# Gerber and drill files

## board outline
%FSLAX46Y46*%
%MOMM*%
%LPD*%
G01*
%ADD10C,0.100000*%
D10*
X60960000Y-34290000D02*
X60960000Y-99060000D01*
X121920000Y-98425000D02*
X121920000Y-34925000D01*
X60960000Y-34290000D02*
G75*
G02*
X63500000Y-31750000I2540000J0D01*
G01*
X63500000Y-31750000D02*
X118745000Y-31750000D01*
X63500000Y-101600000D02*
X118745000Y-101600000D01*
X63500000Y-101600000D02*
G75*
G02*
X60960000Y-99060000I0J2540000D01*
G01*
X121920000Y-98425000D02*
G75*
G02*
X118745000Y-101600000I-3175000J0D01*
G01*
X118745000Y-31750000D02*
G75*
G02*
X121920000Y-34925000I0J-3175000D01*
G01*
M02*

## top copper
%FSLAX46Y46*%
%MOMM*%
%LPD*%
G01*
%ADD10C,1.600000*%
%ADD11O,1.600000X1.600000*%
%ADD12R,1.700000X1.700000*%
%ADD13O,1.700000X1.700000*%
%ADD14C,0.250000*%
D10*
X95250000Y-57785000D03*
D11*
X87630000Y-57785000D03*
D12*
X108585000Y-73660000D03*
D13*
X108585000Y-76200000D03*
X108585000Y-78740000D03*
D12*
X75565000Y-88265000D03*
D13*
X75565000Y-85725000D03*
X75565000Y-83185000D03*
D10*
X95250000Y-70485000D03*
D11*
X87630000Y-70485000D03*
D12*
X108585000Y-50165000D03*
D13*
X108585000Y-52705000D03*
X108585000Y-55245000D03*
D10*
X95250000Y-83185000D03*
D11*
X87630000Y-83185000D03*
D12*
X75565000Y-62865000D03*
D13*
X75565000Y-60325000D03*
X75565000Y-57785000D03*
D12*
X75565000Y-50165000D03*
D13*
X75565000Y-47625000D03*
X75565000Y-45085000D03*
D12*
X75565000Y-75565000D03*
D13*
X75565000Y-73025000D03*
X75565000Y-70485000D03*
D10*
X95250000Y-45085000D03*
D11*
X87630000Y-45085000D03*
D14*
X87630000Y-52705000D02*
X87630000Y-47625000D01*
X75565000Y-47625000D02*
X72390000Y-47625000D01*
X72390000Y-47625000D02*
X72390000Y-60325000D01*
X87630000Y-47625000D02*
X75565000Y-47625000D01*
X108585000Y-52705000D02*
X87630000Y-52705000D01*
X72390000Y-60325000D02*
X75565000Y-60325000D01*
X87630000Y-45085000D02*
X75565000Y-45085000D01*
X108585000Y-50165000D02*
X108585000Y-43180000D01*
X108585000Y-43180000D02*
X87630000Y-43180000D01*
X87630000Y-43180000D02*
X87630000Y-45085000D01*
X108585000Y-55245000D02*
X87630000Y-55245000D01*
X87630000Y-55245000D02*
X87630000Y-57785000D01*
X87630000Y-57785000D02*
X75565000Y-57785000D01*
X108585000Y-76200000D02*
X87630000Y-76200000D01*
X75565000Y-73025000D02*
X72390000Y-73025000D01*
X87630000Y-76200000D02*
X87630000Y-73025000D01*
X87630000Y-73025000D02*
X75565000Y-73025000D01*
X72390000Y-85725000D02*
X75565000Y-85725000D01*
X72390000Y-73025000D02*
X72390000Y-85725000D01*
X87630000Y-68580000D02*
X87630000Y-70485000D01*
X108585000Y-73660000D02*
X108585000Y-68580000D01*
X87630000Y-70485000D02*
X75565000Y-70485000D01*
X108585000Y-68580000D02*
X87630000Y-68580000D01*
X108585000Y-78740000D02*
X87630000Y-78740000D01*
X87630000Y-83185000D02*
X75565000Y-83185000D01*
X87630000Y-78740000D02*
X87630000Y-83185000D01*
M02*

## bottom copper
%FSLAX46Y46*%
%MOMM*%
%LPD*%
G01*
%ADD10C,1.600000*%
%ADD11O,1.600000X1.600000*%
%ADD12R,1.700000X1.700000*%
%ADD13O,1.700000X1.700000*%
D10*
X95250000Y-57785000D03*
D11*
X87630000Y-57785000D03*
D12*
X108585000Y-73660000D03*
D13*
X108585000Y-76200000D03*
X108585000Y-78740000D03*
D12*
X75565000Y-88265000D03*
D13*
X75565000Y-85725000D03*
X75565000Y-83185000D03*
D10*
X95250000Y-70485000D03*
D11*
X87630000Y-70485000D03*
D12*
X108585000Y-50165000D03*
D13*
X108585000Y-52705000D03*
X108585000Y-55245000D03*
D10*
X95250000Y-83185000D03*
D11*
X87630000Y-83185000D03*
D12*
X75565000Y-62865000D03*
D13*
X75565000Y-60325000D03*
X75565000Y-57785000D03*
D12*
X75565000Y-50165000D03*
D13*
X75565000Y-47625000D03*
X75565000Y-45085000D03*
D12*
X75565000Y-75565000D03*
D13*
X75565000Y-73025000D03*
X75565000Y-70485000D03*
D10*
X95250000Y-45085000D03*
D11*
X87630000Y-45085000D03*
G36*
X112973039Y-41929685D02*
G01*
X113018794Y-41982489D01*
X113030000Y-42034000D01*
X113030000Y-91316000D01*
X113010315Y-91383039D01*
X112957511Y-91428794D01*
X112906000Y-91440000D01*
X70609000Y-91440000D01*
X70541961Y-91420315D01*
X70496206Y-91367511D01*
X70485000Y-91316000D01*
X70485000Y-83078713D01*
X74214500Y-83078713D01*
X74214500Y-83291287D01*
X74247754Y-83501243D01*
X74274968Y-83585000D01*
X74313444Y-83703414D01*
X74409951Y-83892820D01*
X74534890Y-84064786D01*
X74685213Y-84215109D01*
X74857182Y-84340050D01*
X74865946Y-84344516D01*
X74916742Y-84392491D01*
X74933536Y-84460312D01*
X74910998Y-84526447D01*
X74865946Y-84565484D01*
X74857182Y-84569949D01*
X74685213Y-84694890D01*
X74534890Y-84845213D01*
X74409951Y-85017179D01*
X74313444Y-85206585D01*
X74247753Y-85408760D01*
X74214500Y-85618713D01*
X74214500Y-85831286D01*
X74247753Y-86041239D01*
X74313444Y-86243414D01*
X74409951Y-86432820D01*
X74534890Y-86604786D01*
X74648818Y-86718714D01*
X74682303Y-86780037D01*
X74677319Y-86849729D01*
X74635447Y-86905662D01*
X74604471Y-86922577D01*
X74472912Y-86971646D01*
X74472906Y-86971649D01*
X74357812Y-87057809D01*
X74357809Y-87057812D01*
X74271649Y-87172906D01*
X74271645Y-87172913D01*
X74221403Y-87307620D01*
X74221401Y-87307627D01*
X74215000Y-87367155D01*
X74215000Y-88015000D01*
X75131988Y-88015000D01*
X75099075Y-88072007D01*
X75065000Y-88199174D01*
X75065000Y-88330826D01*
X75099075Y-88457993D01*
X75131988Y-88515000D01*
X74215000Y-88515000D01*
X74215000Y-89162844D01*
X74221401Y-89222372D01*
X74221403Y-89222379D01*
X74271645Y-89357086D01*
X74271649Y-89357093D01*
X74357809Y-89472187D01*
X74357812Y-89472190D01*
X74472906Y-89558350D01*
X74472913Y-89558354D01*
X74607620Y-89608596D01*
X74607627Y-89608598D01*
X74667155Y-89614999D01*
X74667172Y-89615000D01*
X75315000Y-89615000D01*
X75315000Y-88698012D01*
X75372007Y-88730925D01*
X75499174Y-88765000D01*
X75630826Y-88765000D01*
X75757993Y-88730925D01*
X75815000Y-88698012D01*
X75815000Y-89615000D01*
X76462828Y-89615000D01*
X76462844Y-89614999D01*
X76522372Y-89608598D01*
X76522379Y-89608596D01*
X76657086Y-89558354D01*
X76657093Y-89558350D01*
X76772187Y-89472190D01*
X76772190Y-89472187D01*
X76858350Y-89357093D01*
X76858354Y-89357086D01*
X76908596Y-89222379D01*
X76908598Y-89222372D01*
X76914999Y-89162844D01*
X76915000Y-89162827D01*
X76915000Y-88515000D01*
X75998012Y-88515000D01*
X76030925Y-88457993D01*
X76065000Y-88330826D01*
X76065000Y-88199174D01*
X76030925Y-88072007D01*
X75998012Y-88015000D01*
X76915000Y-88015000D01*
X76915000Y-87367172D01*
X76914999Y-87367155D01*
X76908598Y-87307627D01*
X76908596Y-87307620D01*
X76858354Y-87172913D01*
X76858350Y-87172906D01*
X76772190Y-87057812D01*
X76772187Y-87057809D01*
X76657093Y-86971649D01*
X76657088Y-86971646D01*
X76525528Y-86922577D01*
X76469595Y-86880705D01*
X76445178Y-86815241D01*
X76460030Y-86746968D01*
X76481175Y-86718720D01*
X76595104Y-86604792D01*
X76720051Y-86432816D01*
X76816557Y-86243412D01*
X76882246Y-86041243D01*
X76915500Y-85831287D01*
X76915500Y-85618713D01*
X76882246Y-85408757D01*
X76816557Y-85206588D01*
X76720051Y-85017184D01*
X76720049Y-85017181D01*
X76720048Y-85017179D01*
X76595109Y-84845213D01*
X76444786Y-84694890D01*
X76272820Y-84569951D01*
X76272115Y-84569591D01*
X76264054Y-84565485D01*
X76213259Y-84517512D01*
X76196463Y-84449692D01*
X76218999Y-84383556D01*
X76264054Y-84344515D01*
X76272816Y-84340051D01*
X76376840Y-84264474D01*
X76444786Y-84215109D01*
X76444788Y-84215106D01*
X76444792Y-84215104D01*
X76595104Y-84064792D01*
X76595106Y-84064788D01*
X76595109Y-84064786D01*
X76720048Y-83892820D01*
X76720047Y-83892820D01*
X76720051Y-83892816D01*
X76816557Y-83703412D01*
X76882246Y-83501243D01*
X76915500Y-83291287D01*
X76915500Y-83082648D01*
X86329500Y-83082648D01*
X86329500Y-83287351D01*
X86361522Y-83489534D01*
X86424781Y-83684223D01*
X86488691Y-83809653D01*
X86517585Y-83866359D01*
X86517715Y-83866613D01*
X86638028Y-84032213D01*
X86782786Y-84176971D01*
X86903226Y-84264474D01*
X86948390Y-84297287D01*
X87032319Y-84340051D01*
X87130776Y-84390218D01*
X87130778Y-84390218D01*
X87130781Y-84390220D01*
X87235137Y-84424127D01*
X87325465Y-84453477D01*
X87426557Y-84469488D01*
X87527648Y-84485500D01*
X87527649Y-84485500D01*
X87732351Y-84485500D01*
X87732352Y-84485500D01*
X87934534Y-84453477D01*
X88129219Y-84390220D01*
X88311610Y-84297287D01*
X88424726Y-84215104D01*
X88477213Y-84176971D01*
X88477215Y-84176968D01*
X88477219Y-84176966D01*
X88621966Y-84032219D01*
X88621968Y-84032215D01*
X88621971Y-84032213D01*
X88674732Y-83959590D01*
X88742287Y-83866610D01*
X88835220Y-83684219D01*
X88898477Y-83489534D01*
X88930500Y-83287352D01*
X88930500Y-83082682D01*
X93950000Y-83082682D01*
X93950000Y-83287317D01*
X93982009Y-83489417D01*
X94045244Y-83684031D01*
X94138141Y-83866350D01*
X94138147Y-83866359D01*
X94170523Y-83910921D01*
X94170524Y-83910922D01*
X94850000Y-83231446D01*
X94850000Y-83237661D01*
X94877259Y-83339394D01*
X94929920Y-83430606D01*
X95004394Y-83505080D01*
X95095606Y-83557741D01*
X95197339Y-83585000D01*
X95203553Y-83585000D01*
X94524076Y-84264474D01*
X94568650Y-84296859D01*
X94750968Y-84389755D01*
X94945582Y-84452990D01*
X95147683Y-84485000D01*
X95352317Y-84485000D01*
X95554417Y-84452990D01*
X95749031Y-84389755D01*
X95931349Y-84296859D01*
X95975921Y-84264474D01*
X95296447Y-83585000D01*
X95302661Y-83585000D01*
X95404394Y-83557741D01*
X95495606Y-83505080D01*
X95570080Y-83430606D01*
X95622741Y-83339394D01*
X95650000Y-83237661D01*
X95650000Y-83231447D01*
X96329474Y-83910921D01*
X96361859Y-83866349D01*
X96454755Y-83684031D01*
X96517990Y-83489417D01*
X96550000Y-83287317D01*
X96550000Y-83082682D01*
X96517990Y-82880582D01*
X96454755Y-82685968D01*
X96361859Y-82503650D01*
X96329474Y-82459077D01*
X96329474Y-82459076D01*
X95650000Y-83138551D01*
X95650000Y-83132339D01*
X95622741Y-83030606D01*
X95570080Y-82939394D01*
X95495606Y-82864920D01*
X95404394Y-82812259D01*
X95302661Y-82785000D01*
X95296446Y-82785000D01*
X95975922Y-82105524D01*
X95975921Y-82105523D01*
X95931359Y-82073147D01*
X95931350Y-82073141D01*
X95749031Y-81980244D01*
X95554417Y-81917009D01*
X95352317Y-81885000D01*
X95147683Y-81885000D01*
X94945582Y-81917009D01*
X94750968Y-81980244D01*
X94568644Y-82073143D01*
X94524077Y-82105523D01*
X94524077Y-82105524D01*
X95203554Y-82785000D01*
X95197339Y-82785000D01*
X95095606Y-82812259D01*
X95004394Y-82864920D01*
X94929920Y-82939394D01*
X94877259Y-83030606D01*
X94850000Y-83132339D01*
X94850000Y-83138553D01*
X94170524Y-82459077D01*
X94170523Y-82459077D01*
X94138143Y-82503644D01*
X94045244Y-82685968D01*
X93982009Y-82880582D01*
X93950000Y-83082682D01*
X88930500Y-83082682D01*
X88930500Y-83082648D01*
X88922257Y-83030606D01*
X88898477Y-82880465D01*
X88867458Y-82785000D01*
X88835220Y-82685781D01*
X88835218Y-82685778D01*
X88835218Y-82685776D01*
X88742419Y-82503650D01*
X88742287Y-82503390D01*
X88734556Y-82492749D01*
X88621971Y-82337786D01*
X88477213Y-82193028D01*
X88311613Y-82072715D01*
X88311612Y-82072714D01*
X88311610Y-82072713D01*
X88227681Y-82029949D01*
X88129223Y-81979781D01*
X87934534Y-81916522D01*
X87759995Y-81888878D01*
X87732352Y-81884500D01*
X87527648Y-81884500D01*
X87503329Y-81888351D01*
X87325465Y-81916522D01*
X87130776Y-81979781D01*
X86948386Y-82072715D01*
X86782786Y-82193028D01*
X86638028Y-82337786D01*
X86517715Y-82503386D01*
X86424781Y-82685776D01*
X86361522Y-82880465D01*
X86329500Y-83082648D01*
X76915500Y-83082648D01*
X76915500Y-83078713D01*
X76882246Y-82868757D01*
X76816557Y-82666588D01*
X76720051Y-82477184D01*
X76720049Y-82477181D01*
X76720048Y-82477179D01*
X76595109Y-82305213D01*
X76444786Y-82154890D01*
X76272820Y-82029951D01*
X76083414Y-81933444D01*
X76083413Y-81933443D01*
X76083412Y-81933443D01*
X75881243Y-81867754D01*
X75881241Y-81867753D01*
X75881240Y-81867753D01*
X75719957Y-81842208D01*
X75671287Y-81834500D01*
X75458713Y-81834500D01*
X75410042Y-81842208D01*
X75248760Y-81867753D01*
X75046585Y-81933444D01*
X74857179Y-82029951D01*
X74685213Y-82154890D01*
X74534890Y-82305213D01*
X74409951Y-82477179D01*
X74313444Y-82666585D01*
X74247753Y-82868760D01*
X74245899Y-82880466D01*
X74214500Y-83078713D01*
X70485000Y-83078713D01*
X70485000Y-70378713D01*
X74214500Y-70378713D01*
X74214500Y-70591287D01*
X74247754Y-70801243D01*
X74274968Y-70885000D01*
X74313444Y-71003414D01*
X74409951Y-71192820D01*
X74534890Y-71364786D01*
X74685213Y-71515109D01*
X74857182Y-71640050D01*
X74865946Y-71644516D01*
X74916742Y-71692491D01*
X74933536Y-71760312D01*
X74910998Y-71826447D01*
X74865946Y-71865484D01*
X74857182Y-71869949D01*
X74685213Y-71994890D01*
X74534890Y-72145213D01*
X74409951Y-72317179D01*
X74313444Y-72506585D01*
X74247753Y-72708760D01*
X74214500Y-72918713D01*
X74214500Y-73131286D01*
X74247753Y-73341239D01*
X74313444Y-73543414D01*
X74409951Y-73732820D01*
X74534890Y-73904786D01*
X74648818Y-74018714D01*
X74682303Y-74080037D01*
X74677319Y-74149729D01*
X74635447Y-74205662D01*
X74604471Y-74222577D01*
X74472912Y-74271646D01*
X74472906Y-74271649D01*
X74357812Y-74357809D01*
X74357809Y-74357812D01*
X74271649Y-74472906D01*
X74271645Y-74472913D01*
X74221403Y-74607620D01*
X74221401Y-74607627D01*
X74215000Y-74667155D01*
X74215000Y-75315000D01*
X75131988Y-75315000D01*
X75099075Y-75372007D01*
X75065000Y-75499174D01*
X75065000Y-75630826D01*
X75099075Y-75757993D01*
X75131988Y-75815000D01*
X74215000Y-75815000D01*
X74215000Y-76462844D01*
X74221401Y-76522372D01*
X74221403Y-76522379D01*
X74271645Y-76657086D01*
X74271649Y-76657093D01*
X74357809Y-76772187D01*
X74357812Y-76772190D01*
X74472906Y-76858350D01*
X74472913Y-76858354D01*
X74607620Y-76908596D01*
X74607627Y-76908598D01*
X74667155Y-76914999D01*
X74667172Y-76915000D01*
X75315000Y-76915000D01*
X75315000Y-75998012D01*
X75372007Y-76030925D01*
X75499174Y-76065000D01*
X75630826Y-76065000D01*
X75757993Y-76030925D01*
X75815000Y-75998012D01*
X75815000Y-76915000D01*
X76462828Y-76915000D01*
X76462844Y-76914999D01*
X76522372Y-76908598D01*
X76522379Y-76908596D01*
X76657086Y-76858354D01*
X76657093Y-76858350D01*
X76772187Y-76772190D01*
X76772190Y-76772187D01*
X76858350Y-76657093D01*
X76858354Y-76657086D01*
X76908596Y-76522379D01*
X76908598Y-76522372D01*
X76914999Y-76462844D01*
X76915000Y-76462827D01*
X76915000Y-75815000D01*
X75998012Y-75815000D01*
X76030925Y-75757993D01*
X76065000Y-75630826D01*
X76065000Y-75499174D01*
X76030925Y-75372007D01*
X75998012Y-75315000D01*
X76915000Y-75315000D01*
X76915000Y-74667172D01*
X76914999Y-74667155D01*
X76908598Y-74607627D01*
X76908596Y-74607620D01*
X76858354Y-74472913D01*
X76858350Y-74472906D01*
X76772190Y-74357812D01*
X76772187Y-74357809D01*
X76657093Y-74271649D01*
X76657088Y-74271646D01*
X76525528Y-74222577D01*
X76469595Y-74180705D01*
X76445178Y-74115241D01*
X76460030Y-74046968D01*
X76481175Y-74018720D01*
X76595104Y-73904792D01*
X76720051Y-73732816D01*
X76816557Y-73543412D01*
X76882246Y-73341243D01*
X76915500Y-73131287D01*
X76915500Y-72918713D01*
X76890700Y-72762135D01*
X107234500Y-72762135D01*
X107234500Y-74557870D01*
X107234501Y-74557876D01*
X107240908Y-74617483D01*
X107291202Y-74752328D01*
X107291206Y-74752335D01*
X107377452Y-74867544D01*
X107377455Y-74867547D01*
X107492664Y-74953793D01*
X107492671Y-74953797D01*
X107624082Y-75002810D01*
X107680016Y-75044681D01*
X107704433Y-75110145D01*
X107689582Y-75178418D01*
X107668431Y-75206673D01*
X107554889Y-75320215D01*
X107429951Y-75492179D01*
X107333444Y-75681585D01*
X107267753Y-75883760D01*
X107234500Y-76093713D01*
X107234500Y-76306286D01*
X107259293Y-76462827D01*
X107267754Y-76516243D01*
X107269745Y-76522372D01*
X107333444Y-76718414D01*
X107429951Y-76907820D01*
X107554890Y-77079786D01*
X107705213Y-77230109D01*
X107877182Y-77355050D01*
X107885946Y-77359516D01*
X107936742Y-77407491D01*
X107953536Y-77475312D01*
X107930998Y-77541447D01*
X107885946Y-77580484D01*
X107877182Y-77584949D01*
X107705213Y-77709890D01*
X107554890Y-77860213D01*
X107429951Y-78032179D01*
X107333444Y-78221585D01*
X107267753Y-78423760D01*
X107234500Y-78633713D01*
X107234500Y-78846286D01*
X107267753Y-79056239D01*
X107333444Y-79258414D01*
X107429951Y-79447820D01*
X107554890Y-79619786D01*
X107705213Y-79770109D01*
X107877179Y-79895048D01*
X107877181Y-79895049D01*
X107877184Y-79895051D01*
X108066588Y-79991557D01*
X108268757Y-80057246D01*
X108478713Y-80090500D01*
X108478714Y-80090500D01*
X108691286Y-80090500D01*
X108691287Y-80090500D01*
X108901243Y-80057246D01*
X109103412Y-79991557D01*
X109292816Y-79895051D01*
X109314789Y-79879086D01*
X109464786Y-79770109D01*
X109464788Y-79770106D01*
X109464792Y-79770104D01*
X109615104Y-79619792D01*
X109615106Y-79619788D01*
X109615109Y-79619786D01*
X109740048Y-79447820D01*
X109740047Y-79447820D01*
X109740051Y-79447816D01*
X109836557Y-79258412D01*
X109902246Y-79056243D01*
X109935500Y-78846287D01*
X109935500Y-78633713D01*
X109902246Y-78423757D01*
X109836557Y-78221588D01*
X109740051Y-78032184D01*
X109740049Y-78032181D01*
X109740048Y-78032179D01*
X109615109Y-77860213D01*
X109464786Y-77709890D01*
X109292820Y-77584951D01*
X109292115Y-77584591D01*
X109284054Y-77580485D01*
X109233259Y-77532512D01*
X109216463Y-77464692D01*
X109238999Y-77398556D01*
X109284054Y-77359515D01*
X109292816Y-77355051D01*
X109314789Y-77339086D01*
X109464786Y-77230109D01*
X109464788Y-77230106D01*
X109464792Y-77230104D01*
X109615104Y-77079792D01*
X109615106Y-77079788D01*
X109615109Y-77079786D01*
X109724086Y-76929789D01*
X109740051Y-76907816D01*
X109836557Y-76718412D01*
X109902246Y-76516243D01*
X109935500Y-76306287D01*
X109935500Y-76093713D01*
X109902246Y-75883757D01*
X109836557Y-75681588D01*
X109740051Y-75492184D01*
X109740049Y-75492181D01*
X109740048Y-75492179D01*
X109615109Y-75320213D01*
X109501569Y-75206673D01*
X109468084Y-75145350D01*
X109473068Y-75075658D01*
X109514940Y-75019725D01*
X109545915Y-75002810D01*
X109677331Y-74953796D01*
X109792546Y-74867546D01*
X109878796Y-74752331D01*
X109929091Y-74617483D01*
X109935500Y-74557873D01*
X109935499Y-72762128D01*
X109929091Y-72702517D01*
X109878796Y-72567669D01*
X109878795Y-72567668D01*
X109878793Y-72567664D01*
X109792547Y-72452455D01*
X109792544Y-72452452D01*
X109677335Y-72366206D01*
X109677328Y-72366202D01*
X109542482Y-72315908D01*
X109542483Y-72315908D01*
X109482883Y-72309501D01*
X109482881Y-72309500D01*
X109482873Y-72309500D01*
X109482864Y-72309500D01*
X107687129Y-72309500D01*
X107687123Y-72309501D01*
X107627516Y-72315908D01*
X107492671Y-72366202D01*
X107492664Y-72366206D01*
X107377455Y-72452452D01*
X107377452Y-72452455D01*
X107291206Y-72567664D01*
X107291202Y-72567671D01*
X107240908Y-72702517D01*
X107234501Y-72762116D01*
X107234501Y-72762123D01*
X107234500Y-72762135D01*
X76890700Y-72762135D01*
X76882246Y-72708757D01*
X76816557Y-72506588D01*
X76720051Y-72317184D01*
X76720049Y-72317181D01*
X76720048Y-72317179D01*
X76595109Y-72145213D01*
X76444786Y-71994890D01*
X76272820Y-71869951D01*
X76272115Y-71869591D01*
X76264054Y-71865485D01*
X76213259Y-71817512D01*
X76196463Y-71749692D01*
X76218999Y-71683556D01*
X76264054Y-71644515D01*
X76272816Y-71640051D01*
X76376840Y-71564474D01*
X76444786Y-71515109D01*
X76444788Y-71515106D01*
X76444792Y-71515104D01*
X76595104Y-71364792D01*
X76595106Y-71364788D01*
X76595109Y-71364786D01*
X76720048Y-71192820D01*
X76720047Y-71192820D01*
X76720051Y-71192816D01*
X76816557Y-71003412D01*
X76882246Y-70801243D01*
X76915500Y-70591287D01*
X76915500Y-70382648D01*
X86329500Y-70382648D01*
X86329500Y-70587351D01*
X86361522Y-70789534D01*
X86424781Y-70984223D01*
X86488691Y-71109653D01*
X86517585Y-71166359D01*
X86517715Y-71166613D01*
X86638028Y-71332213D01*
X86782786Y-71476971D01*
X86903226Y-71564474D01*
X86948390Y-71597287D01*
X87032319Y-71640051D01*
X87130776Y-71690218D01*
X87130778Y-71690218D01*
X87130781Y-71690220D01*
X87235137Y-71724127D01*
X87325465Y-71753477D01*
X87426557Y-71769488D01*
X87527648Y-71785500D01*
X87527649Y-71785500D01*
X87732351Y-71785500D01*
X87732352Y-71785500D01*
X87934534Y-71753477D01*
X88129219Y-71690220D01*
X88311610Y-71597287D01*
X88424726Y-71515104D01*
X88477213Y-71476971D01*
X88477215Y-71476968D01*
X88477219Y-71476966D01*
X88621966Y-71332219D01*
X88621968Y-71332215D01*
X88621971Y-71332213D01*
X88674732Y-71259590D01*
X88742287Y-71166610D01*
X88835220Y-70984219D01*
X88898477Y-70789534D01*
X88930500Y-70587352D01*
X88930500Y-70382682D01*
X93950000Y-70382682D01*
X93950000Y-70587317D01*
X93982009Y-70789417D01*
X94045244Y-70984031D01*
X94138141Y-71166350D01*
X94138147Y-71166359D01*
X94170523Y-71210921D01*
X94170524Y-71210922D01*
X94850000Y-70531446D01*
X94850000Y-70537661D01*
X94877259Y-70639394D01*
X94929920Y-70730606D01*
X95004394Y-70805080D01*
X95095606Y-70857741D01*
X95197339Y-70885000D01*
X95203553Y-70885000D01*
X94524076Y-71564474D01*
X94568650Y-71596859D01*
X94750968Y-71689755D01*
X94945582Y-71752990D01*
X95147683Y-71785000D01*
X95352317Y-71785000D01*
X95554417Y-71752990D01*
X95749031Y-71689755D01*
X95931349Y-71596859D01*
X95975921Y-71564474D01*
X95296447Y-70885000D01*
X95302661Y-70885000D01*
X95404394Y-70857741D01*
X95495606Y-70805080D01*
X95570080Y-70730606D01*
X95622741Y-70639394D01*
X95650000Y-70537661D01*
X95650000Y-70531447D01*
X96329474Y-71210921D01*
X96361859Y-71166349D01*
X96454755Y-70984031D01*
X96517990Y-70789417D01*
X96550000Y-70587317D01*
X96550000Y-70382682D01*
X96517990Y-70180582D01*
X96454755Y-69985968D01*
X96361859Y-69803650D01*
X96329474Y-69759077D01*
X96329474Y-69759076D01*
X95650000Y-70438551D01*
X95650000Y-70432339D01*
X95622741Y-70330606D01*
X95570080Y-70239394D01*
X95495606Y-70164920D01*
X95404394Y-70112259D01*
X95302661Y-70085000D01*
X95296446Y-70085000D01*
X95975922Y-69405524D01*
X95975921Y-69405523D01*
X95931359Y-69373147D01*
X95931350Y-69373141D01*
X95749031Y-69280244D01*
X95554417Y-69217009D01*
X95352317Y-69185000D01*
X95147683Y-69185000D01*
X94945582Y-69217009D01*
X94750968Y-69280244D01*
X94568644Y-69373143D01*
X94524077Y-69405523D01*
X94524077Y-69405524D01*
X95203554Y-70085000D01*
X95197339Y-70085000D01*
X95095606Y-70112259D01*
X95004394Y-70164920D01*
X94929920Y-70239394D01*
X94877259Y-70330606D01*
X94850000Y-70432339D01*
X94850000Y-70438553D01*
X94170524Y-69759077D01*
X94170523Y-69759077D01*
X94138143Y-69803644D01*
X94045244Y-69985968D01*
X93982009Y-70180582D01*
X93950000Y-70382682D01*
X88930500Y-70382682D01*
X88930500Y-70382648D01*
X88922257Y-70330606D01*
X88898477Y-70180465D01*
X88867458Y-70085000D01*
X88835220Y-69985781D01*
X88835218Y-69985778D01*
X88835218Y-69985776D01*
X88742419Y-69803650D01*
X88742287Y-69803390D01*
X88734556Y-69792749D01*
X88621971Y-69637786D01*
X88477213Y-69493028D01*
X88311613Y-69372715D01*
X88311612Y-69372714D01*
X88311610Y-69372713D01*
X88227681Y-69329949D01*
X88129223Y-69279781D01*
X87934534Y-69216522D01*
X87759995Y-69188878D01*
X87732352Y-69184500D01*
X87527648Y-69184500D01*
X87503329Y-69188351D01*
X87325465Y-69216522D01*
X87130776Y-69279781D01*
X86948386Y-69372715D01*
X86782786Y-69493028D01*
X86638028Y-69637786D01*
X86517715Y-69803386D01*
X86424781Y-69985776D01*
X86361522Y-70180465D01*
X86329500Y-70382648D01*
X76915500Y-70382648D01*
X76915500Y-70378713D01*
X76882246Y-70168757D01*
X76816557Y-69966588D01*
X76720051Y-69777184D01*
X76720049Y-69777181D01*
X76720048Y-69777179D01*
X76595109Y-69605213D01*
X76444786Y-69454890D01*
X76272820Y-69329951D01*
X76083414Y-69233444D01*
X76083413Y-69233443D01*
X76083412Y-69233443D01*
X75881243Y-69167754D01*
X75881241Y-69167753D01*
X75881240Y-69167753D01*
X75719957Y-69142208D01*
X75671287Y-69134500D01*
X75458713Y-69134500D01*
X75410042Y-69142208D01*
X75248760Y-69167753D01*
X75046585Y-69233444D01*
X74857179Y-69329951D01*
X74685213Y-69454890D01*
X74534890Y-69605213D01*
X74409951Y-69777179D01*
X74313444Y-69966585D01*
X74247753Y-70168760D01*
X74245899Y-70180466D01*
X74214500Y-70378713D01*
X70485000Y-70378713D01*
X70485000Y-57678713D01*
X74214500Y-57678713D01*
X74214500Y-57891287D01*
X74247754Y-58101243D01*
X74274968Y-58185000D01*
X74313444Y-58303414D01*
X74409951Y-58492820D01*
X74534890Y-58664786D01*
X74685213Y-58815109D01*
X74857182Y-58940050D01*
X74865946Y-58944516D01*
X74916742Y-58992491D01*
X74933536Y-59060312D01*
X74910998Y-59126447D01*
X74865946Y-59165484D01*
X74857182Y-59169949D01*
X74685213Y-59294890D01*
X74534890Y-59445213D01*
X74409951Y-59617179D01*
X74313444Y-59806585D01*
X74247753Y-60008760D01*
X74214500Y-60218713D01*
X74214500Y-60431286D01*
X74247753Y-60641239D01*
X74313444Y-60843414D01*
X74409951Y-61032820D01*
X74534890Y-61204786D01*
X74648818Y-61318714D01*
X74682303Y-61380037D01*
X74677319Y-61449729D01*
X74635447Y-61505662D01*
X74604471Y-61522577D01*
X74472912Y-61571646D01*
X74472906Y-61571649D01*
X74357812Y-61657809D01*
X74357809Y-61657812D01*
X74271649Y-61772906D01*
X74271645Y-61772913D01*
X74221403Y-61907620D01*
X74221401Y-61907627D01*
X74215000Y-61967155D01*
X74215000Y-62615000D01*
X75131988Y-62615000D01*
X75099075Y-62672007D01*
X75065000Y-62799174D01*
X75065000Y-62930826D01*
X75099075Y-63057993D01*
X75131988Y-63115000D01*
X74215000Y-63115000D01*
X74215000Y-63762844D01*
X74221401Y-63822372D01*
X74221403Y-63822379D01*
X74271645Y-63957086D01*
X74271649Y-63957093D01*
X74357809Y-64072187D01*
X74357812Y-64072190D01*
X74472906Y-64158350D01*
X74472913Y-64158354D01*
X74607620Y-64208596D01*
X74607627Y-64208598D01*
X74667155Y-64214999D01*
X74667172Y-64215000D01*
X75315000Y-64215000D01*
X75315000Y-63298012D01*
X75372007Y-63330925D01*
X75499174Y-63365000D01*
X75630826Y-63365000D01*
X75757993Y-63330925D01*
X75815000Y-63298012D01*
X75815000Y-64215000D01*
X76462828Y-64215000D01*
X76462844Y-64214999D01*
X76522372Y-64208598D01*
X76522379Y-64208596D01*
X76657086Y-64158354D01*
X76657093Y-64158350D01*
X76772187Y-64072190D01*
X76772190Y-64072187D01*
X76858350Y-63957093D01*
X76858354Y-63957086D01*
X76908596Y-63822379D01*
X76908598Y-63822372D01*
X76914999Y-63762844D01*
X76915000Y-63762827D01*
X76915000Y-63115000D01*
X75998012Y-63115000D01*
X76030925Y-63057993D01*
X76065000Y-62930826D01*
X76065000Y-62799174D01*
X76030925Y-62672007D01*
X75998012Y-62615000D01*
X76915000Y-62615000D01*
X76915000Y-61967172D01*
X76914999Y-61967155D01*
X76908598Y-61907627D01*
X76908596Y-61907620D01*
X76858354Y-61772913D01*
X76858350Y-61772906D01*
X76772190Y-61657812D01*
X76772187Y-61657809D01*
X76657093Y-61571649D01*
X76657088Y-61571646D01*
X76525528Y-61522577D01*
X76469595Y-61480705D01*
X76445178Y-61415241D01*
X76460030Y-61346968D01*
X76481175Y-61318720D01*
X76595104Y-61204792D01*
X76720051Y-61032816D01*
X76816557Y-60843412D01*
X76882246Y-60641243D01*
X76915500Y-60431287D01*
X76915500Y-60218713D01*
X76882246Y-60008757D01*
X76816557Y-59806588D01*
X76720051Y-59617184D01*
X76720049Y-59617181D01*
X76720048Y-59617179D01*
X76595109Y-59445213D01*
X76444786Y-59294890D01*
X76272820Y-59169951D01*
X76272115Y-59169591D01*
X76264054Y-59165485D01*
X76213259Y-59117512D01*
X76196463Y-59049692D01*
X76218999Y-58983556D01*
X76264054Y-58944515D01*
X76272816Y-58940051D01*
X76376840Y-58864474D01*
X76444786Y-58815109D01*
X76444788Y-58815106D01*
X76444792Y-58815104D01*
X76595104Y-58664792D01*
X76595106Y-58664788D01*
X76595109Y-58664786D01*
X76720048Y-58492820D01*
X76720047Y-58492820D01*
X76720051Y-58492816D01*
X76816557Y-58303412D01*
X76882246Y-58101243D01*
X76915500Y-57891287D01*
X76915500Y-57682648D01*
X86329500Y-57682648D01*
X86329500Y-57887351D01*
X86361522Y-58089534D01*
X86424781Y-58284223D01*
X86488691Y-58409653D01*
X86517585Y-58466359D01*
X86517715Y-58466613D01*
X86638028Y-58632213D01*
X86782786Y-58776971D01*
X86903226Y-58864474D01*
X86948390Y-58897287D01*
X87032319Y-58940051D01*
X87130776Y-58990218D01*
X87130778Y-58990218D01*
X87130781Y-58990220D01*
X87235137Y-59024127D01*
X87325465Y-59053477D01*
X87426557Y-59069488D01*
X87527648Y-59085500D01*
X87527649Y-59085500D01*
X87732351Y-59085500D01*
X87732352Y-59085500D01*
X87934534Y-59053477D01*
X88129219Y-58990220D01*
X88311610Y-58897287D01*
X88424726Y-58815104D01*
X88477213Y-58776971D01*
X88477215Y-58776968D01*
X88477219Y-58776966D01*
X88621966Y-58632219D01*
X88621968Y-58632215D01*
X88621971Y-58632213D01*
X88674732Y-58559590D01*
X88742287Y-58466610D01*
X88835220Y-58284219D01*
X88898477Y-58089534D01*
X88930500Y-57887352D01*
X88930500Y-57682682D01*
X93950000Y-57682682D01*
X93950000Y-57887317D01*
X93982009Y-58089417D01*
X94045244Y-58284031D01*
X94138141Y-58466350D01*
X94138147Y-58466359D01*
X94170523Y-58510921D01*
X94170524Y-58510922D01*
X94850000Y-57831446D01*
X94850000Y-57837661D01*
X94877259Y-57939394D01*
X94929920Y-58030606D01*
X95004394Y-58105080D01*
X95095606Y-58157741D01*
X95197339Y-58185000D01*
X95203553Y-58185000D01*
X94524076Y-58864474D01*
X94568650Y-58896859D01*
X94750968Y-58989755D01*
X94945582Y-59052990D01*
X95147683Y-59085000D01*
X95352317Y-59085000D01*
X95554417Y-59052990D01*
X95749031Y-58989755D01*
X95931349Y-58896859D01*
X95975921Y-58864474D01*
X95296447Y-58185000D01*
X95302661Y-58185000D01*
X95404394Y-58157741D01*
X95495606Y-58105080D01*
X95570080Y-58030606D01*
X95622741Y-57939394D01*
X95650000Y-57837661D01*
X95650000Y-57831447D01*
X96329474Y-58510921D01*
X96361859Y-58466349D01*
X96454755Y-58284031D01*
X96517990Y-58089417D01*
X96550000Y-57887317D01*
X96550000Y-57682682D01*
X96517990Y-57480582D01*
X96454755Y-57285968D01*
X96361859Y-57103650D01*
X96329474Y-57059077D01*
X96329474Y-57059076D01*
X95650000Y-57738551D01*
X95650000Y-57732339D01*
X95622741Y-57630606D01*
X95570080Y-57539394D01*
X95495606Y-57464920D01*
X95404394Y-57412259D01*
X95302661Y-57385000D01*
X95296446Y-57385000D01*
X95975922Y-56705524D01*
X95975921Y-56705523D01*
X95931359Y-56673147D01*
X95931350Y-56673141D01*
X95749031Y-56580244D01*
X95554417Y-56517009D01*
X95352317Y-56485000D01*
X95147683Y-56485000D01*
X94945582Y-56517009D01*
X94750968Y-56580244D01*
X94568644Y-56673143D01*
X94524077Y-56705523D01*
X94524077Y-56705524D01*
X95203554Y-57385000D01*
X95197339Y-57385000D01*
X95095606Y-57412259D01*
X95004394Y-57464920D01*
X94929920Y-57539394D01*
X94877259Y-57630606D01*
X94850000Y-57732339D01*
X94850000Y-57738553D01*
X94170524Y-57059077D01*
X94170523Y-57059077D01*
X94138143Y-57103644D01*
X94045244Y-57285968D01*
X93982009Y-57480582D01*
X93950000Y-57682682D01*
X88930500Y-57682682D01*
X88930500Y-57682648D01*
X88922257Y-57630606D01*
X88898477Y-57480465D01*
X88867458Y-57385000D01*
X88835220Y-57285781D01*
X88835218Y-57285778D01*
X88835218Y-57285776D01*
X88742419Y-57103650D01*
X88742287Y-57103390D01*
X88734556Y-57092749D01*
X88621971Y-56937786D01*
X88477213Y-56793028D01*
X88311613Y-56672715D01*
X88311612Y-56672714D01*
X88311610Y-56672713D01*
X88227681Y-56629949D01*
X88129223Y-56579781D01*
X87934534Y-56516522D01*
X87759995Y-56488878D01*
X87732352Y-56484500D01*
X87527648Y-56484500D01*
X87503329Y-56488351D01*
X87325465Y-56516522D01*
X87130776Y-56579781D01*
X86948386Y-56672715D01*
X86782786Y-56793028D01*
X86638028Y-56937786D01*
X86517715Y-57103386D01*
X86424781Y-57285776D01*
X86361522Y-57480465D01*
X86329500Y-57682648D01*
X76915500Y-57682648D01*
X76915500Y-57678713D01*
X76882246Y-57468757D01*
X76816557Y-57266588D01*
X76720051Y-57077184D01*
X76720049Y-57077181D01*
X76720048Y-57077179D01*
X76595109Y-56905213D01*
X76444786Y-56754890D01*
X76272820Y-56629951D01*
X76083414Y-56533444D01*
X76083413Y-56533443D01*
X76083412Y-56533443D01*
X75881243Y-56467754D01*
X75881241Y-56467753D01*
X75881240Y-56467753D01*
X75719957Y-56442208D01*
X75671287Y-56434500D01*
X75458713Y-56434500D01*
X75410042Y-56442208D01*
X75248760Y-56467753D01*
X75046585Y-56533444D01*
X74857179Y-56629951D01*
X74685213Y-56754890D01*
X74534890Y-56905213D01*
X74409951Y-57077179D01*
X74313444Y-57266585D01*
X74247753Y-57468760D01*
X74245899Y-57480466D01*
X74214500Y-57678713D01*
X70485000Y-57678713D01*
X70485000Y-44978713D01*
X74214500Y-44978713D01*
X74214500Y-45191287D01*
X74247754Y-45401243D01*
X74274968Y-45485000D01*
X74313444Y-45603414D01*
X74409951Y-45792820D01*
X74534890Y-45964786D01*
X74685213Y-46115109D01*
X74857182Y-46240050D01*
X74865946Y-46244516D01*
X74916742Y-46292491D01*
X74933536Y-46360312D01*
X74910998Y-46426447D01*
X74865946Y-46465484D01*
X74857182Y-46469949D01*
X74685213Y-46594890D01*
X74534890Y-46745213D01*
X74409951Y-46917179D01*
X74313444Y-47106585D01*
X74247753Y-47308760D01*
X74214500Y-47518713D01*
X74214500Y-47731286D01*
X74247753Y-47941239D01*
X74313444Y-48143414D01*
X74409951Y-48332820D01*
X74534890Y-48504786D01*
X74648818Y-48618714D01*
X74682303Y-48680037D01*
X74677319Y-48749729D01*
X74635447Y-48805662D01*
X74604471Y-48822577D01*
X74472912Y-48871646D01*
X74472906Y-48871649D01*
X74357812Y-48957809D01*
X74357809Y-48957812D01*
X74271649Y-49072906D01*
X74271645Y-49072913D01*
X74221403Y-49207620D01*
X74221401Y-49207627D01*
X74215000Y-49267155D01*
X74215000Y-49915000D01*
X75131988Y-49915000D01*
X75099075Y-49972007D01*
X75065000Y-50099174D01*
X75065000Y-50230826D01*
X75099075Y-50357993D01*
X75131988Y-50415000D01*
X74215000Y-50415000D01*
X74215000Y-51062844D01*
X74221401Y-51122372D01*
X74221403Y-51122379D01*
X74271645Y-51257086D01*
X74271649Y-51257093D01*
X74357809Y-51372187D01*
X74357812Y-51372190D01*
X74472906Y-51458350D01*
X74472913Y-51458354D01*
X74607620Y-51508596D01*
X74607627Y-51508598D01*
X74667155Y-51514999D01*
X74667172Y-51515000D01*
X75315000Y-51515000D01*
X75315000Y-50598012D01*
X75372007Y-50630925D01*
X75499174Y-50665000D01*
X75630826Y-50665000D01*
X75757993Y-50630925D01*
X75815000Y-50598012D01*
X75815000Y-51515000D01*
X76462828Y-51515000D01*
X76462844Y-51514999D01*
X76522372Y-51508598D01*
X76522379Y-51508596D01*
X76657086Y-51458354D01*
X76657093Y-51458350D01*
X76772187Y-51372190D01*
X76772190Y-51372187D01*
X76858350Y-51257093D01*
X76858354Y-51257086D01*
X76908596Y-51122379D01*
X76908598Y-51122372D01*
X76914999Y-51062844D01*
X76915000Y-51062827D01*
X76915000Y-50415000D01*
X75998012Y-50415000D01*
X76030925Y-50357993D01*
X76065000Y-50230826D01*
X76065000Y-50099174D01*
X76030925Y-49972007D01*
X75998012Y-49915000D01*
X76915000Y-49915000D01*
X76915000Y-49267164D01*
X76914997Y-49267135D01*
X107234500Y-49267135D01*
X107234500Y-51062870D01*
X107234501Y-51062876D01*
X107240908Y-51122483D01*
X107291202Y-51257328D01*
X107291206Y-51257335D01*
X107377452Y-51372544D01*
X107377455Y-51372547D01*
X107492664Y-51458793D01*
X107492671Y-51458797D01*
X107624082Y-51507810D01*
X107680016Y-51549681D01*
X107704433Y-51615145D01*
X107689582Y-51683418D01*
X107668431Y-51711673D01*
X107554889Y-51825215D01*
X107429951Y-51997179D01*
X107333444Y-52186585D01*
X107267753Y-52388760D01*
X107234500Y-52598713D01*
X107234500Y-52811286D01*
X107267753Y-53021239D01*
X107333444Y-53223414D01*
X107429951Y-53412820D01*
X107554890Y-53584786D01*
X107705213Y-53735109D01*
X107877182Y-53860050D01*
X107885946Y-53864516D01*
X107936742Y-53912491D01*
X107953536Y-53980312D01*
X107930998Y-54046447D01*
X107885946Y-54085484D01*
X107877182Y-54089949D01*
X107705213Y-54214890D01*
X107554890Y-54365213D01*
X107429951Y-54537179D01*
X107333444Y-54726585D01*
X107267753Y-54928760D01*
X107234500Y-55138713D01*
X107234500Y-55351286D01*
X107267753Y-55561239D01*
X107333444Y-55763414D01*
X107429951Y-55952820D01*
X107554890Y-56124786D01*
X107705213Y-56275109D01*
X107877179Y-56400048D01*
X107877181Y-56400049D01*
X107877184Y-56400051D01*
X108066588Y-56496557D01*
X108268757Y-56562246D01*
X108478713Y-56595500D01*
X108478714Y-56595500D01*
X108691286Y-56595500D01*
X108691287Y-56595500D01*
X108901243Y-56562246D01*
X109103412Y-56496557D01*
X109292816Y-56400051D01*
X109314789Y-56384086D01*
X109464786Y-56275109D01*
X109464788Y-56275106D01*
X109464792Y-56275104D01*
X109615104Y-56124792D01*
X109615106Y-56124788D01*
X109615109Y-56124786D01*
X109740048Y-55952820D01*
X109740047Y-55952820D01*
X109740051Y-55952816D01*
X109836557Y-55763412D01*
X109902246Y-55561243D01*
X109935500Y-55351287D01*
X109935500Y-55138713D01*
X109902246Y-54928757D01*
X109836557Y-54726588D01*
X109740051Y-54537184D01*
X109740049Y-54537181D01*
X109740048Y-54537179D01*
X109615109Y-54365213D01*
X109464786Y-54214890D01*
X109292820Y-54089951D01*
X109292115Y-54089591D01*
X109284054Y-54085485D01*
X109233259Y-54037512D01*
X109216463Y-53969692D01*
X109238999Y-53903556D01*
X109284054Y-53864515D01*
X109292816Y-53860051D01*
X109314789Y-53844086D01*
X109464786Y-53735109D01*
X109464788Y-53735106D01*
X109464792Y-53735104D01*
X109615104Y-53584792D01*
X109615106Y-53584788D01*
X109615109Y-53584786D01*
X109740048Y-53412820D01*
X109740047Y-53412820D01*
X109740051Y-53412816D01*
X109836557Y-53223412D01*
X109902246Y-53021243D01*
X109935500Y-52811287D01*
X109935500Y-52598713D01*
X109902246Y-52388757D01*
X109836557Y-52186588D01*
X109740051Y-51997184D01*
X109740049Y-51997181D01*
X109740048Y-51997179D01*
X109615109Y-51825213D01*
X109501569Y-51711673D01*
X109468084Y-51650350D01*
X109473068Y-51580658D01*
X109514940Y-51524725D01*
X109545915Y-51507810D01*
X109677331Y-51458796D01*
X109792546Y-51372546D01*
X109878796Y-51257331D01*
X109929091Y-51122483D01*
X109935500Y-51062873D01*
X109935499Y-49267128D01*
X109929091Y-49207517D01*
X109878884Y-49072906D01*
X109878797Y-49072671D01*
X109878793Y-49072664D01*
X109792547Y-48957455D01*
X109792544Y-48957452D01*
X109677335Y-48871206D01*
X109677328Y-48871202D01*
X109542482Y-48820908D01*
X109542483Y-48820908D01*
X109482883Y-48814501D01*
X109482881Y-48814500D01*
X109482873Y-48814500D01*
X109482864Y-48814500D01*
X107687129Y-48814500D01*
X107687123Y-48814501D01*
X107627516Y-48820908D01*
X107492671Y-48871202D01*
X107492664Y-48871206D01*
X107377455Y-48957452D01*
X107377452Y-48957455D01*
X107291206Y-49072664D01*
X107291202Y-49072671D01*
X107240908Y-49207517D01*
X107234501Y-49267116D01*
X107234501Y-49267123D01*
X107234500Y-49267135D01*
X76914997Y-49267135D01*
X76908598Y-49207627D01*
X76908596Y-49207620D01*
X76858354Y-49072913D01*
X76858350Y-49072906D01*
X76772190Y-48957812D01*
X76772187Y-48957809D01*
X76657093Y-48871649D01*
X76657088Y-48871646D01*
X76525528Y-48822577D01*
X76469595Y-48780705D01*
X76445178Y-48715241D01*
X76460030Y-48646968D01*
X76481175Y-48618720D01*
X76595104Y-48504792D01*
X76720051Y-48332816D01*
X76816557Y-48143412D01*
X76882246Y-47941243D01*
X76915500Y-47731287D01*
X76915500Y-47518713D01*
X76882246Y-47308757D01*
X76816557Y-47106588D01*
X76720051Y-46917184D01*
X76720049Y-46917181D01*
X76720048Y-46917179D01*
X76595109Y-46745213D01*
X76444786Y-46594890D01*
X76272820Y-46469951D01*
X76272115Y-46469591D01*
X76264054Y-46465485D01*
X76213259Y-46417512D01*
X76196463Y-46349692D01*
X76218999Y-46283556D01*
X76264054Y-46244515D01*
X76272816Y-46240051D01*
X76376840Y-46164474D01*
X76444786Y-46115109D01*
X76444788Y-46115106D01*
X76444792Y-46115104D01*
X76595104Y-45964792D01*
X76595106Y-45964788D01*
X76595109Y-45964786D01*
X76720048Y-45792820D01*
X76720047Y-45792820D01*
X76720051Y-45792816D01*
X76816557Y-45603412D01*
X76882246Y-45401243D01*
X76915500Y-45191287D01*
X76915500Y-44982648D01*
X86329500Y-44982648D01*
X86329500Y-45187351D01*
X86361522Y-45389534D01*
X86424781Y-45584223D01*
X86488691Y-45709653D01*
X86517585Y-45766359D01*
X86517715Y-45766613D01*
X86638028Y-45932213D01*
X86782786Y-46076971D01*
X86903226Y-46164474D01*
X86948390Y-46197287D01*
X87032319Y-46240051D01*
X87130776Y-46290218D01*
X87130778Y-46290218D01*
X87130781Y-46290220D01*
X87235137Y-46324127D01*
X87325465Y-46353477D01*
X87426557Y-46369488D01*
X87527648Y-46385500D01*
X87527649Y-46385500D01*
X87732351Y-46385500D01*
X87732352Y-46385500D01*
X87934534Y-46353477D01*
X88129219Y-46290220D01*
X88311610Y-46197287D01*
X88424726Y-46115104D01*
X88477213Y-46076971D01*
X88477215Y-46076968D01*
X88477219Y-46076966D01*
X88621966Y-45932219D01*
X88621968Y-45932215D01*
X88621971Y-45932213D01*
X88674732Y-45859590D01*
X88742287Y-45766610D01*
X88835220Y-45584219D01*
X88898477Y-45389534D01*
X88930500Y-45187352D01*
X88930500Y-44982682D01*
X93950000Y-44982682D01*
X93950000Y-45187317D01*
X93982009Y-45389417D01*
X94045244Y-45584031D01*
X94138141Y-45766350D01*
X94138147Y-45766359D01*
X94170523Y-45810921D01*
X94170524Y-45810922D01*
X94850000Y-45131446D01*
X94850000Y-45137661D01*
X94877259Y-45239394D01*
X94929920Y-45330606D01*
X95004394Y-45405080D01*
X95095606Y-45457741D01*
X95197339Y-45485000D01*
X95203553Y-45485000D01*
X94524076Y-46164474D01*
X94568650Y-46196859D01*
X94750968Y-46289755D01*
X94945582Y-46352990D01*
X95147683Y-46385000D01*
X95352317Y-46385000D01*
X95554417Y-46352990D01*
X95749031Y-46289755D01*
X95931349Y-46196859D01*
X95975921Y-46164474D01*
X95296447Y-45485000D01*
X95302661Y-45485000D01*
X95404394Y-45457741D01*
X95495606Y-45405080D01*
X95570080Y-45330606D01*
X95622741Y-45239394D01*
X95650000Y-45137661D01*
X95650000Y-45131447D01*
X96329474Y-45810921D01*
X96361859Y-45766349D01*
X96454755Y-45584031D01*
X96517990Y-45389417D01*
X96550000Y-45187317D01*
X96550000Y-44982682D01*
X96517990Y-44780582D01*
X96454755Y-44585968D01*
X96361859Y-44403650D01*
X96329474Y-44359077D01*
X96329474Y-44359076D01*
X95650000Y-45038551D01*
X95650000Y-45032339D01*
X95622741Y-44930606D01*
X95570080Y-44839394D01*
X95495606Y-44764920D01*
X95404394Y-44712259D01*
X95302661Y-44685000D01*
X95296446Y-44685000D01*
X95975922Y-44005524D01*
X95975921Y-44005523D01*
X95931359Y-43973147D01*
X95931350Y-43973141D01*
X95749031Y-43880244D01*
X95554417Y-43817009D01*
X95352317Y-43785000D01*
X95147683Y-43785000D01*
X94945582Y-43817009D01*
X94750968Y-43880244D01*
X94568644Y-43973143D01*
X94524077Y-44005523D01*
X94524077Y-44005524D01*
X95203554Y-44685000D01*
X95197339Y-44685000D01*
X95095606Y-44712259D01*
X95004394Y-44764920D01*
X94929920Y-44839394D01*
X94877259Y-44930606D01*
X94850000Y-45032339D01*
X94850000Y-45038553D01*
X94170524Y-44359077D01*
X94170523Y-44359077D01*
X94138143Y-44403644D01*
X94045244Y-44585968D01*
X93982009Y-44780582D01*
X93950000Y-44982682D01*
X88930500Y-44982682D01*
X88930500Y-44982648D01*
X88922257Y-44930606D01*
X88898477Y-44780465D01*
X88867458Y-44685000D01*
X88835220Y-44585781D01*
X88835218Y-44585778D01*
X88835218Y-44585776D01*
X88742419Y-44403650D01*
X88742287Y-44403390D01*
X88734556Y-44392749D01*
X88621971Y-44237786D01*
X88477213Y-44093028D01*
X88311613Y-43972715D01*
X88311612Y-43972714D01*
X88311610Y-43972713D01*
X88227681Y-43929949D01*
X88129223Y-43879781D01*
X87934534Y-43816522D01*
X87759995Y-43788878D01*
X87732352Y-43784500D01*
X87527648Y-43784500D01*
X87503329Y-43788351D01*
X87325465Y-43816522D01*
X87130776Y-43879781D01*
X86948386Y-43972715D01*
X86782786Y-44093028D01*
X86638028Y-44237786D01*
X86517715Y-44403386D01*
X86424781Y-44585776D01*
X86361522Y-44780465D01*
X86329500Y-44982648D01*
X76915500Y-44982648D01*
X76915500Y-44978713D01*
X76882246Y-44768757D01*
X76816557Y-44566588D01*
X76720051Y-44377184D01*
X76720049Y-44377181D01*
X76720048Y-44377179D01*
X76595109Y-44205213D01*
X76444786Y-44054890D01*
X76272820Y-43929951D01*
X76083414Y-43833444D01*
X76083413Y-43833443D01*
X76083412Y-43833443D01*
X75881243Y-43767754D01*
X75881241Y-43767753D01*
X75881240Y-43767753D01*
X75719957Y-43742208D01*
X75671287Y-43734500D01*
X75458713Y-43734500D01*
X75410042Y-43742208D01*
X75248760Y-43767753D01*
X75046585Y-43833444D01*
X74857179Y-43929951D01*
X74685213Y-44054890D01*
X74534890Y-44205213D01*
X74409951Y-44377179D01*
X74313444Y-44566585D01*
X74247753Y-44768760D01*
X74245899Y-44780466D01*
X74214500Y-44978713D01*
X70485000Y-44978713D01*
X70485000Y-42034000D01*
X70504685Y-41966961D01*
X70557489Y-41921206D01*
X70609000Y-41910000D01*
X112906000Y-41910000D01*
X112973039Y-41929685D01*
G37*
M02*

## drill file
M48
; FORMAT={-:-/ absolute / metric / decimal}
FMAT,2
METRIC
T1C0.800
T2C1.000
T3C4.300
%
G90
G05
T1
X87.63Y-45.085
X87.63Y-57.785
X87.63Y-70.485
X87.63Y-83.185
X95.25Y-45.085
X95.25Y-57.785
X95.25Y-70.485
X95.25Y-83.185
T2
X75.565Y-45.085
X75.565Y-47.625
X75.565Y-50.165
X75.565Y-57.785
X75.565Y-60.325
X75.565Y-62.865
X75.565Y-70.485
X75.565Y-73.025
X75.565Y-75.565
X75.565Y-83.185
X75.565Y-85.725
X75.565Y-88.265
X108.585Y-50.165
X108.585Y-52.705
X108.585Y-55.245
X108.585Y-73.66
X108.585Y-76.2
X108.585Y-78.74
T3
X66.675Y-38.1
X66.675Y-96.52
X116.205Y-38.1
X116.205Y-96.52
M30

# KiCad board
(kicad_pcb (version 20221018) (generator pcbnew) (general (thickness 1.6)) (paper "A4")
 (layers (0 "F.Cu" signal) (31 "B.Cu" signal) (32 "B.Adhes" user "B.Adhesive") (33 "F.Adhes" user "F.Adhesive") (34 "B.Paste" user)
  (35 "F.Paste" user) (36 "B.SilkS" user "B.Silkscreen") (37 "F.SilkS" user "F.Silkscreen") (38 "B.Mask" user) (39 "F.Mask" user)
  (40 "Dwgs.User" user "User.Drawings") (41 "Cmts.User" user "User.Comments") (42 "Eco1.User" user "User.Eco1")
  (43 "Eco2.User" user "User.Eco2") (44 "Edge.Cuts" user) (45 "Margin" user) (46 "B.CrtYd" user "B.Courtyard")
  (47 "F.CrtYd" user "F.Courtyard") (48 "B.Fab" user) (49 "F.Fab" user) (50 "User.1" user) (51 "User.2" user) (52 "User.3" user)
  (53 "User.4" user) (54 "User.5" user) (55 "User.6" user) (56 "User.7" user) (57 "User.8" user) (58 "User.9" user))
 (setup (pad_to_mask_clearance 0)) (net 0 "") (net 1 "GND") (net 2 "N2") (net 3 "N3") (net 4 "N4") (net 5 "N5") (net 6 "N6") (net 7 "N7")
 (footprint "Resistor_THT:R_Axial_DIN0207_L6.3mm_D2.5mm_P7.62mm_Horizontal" (layer "F.Cu") (at 95.25 57.785 180)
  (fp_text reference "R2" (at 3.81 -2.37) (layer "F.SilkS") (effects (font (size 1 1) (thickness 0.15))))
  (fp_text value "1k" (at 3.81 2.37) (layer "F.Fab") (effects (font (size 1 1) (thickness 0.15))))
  (pad "1" thru_hole circle (at 0 0 180) (size 1.6 1.6) (drill 0.8) (layers "*.Cu" "*.Mask") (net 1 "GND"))
  (pad "2" thru_hole oval (at 7.62 0 180) (size 1.6 1.6) (drill 0.8) (layers "*.Cu" "*.Mask") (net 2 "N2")))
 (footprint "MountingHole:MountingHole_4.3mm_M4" (layer "F.Cu") (at 66.675 38.1)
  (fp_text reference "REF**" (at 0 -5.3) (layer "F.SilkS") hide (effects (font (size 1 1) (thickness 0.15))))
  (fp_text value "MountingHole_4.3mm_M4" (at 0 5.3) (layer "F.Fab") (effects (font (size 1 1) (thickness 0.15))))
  (pad "" np_thru_hole circle (at 0 0) (size 4.3 4.3) (drill 4.3) (layers "*.Cu" "*.Mask")))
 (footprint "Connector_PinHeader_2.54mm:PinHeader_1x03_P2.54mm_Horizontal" (layer "F.Cu") (at 108.585 73.66)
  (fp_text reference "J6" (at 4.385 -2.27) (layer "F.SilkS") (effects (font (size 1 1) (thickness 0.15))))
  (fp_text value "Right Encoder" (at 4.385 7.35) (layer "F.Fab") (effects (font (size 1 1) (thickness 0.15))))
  (pad "1" thru_hole rect (at 0 0) (size 1.7 1.7) (drill 1) (layers "*.Cu" "*.Mask") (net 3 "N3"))
  (pad "2" thru_hole oval (at 0 2.54) (size 1.7 1.7) (drill 1) (layers "*.Cu" "*.Mask") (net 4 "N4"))
  (pad "3" thru_hole oval (at 0 5.08) (size 1.7 1.7) (drill 1) (layers "*.Cu" "*.Mask") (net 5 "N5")))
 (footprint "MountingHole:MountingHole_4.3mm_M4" (layer "F.Cu") (at 66.675 96.52)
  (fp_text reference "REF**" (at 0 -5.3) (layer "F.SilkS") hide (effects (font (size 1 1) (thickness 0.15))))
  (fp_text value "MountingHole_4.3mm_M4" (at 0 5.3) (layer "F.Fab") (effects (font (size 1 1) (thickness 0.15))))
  (pad "" np_thru_hole circle (at 0 0) (size 4.3 4.3) (drill 4.3) (layers "*.Cu" "*.Mask")))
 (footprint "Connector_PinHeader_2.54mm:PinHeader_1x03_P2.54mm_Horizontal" (layer "F.Cu") (at 75.565 88.265 180)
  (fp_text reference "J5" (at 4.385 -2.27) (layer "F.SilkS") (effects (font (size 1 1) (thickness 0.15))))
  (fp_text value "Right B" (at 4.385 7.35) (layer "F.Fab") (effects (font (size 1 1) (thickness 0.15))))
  (pad "1" thru_hole rect (at 0 0 180) (size 1.7 1.7) (drill 1) (layers "*.Cu" "*.Mask") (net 1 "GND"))
  (pad "2" thru_hole oval (at 0 2.54 180) (size 1.7 1.7) (drill 1) (layers "*.Cu" "*.Mask") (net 4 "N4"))
  (pad "3" thru_hole oval (at 0 5.08 180) (size 1.7 1.7) (drill 1) (layers "*.Cu" "*.Mask") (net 5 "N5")))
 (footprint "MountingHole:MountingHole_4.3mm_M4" (layer "F.Cu") (at 116.205 38.1)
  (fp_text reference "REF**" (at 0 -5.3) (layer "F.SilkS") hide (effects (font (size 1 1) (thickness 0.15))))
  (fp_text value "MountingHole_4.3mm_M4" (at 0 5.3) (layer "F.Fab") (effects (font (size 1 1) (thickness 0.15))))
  (pad "" np_thru_hole circle (at 0 0) (size 4.3 4.3) (drill 4.3) (layers "*.Cu" "*.Mask")))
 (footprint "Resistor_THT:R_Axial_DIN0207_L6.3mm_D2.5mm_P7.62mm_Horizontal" (layer "F.Cu") (at 95.25 70.485 180)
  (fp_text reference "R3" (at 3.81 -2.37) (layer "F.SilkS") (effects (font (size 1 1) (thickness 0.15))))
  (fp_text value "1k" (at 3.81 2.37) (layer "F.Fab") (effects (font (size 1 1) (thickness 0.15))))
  (pad "1" thru_hole circle (at 0 0 180) (size 1.6 1.6) (drill 0.8) (layers "*.Cu" "*.Mask") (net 1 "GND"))
  (pad "2" thru_hole oval (at 7.62 0 180) (size 1.6 1.6) (drill 0.8) (layers "*.Cu" "*.Mask") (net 3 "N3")))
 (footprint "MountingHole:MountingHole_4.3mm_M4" (layer "F.Cu") (at 116.205 96.52)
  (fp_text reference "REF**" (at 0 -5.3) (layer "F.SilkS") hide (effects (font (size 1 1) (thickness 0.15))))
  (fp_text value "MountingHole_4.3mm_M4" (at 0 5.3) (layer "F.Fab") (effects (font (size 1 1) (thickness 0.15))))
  (pad "" np_thru_hole circle (at 0 0) (size 4.3 4.3) (drill 4.3) (layers "*.Cu" "*.Mask")))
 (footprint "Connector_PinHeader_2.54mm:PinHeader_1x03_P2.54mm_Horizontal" (layer "F.Cu") (at 108.585 50.165)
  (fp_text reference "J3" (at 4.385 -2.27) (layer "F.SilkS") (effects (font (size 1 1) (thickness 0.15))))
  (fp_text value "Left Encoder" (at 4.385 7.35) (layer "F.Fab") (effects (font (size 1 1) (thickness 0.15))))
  (pad "1" thru_hole rect (at 0 0) (size 1.7 1.7) (drill 1) (layers "*.Cu" "*.Mask") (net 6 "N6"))
  (pad "2" thru_hole oval (at 0 2.54) (size 1.7 1.7) (drill 1) (layers "*.Cu" "*.Mask") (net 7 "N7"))
  (pad "3" thru_hole oval (at 0 5.08) (size 1.7 1.7) (drill 1) (layers "*.Cu" "*.Mask") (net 2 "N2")))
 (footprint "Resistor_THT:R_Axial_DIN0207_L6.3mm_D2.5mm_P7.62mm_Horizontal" (layer "F.Cu") (at 95.25 83.185 180)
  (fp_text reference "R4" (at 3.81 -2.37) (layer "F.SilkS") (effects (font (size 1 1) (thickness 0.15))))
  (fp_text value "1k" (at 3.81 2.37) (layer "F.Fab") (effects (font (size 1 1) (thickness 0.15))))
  (pad "1" thru_hole circle (at 0 0 180) (size 1.6 1.6) (drill 0.8) (layers "*.Cu" "*.Mask") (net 1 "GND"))
  (pad "2" thru_hole oval (at 7.62 0 180) (size 1.6 1.6) (drill 0.8) (layers "*.Cu" "*.Mask") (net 5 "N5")))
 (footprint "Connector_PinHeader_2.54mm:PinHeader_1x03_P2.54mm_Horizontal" (layer "F.Cu") (at 75.565 62.865 180)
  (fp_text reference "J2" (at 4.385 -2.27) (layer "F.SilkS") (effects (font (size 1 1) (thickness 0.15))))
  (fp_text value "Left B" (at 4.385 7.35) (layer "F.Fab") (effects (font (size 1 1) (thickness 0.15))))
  (pad "1" thru_hole rect (at 0 0 180) (size 1.7 1.7) (drill 1) (layers "*.Cu" "*.Mask") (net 1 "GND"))
  (pad "2" thru_hole oval (at 0 2.54 180) (size 1.7 1.7) (drill 1) (layers "*.Cu" "*.Mask") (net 7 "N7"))
  (pad "3" thru_hole oval (at 0 5.08 180) (size 1.7 1.7) (drill 1) (layers "*.Cu" "*.Mask") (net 2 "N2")))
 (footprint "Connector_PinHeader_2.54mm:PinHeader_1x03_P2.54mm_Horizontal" (layer "F.Cu") (at 75.565 50.165 180)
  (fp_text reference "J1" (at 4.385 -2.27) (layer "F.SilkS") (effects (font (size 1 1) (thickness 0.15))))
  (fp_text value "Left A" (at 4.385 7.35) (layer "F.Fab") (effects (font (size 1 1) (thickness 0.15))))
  (pad "1" thru_hole rect (at 0 0 180) (size 1.7 1.7) (drill 1) (layers "*.Cu" "*.Mask") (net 1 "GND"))
  (pad "2" thru_hole oval (at 0 2.54 180) (size 1.7 1.7) (drill 1) (layers "*.Cu" "*.Mask") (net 7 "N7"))
  (pad "3" thru_hole oval (at 0 5.08 180) (size 1.7 1.7) (drill 1) (layers "*.Cu" "*.Mask") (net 6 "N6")))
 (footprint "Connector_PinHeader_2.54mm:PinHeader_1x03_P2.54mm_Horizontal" (layer "F.Cu") (at 75.565 75.565 180)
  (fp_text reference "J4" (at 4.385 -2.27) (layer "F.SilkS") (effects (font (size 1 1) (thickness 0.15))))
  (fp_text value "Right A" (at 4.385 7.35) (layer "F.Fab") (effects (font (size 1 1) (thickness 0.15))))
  (pad "1" thru_hole rect (at 0 0 180) (size 1.7 1.7) (drill 1) (layers "*.Cu" "*.Mask") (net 1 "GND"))
  (pad "2" thru_hole oval (at 0 2.54 180) (size 1.7 1.7) (drill 1) (layers "*.Cu" "*.Mask") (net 4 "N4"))
  (pad "3" thru_hole oval (at 0 5.08 180) (size 1.7 1.7) (drill 1) (layers "*.Cu" "*.Mask") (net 3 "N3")))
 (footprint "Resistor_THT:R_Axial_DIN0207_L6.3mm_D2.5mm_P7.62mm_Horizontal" (layer "F.Cu") (at 95.25 45.085 180)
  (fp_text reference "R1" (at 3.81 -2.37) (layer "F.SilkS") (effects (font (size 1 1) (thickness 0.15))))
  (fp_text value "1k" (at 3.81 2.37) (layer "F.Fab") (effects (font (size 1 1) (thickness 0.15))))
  (pad "1" thru_hole circle (at 0 0 180) (size 1.6 1.6) (drill 0.8) (layers "*.Cu" "*.Mask") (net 1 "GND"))
  (pad "2" thru_hole oval (at 7.62 0 180) (size 1.6 1.6) (drill 0.8) (layers "*.Cu" "*.Mask") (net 6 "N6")))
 (gr_line (start 60.96 34.29) (end 60.96 99.06) (stroke (width 0.1) (type default)) (layer "Edge.Cuts"))
 (gr_line (start 121.92 98.425) (end 121.92 34.925) (stroke (width 0.1) (type default)) (layer "Edge.Cuts"))
 (gr_arc (start 60.96 34.29) (mid 61.703949 32.493949) (end 63.5 31.75) (stroke (width 0.1) (type default)) (layer "Edge.Cuts"))
 (gr_line (start 63.5 31.75) (end 118.745 31.75) (stroke (width 0.1) (type default)) (layer "Edge.Cuts"))
 (gr_line (start 63.5 101.6) (end 118.745 101.6) (stroke (width 0.1) (type default)) (layer "Edge.Cuts"))
 (gr_arc (start 63.5 101.6) (mid 61.703949 100.856051) (end 60.96 99.06) (stroke (width 0.1) (type default)) (layer "Edge.Cuts"))
 (gr_arc (start 121.92 98.425) (mid 120.990064 100.670064) (end 118.745 101.6) (stroke (width 0.1) (type default)) (layer "Edge.Cuts"))
 (gr_arc (start 118.745 31.75) (mid 120.990064 32.679936) (end 121.92 34.925) (stroke (width 0.1) (type default)) (layer "Edge.Cuts"))
 (segment (start 87.63 52.705) (end 87.63 47.625) (width 0.25) (layer "F.Cu") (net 7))
 (segment (start 75.565 47.625) (end 72.39 47.625) (width 0.25) (layer "F.Cu") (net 7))
 (segment (start 72.39 47.625) (end 72.39 60.325) (width 0.25) (layer "F.Cu") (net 7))
 (segment (start 87.63 47.625) (end 75.565 47.625) (width 0.25) (layer "F.Cu") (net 7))
 (segment (start 108.585 52.705) (end 87.63 52.705) (width 0.25) (layer "F.Cu") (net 7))
 (segment (start 72.39 60.325) (end 75.565 60.325) (width 0.25) (layer "F.Cu") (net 7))
 (segment (start 87.63 45.085) (end 75.565 45.085) (width 0.25) (layer "F.Cu") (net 6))
 (segment (start 108.585 50.165) (end 108.585 43.18) (width 0.25) (layer "F.Cu") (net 6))
 (segment (start 108.585 43.18) (end 87.63 43.18) (width 0.25) (layer "F.Cu") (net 6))
 (segment (start 87.63 43.18) (end 87.63 45.085) (width 0.25) (layer "F.Cu") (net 6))
 (segment (start 108.585 55.245) (end 87.63 55.245) (width 0.25) (layer "F.Cu") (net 2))
 (segment (start 87.63 55.245) (end 87.63 57.785) (width 0.25) (layer "F.Cu") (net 2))
 (segment (start 87.63 57.785) (end 75.565 57.785) (width 0.25) (layer "F.Cu") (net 2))
 (segment (start 108.585 76.2) (end 87.63 76.2) (width 0.25) (layer "F.Cu") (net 4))
 (segment (start 75.565 73.025) (end 72.39 73.025) (width 0.25) (layer "F.Cu") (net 4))
 (segment (start 87.63 76.2) (end 87.63 73.025) (width 0.25) (layer "F.Cu") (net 4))
 (segment (start 87.63 73.025) (end 75.565 73.025) (width 0.25) (layer "F.Cu") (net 4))
 (segment (start 72.39 85.725) (end 75.565 85.725) (width 0.25) (layer "F.Cu") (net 4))
 (segment (start 72.39 73.025) (end 72.39 85.725) (width 0.25) (layer "F.Cu") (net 4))
 (segment (start 87.63 68.58) (end 87.63 70.485) (width 0.25) (layer "F.Cu") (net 3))
 (segment (start 108.585 73.66) (end 108.585 68.58) (width 0.25) (layer "F.Cu") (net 3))
 (segment (start 87.63 70.485) (end 75.565 70.485) (width 0.25) (layer "F.Cu") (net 3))
 (segment (start 108.585 68.58) (end 87.63 68.58) (width 0.25) (layer "F.Cu") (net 3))
 (segment (start 108.585 78.74) (end 87.63 78.74) (width 0.25) (layer "F.Cu") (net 5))
 (segment (start 87.63 83.185) (end 75.565 83.185) (width 0.25) (layer "F.Cu") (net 5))
 (segment (start 87.63 78.74) (end 87.63 83.185) (width 0.25) (layer "F.Cu") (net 5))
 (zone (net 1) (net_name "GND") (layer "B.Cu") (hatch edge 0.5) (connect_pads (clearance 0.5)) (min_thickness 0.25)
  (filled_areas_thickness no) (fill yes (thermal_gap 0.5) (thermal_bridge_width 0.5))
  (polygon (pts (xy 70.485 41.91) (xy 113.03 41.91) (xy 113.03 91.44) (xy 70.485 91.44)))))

